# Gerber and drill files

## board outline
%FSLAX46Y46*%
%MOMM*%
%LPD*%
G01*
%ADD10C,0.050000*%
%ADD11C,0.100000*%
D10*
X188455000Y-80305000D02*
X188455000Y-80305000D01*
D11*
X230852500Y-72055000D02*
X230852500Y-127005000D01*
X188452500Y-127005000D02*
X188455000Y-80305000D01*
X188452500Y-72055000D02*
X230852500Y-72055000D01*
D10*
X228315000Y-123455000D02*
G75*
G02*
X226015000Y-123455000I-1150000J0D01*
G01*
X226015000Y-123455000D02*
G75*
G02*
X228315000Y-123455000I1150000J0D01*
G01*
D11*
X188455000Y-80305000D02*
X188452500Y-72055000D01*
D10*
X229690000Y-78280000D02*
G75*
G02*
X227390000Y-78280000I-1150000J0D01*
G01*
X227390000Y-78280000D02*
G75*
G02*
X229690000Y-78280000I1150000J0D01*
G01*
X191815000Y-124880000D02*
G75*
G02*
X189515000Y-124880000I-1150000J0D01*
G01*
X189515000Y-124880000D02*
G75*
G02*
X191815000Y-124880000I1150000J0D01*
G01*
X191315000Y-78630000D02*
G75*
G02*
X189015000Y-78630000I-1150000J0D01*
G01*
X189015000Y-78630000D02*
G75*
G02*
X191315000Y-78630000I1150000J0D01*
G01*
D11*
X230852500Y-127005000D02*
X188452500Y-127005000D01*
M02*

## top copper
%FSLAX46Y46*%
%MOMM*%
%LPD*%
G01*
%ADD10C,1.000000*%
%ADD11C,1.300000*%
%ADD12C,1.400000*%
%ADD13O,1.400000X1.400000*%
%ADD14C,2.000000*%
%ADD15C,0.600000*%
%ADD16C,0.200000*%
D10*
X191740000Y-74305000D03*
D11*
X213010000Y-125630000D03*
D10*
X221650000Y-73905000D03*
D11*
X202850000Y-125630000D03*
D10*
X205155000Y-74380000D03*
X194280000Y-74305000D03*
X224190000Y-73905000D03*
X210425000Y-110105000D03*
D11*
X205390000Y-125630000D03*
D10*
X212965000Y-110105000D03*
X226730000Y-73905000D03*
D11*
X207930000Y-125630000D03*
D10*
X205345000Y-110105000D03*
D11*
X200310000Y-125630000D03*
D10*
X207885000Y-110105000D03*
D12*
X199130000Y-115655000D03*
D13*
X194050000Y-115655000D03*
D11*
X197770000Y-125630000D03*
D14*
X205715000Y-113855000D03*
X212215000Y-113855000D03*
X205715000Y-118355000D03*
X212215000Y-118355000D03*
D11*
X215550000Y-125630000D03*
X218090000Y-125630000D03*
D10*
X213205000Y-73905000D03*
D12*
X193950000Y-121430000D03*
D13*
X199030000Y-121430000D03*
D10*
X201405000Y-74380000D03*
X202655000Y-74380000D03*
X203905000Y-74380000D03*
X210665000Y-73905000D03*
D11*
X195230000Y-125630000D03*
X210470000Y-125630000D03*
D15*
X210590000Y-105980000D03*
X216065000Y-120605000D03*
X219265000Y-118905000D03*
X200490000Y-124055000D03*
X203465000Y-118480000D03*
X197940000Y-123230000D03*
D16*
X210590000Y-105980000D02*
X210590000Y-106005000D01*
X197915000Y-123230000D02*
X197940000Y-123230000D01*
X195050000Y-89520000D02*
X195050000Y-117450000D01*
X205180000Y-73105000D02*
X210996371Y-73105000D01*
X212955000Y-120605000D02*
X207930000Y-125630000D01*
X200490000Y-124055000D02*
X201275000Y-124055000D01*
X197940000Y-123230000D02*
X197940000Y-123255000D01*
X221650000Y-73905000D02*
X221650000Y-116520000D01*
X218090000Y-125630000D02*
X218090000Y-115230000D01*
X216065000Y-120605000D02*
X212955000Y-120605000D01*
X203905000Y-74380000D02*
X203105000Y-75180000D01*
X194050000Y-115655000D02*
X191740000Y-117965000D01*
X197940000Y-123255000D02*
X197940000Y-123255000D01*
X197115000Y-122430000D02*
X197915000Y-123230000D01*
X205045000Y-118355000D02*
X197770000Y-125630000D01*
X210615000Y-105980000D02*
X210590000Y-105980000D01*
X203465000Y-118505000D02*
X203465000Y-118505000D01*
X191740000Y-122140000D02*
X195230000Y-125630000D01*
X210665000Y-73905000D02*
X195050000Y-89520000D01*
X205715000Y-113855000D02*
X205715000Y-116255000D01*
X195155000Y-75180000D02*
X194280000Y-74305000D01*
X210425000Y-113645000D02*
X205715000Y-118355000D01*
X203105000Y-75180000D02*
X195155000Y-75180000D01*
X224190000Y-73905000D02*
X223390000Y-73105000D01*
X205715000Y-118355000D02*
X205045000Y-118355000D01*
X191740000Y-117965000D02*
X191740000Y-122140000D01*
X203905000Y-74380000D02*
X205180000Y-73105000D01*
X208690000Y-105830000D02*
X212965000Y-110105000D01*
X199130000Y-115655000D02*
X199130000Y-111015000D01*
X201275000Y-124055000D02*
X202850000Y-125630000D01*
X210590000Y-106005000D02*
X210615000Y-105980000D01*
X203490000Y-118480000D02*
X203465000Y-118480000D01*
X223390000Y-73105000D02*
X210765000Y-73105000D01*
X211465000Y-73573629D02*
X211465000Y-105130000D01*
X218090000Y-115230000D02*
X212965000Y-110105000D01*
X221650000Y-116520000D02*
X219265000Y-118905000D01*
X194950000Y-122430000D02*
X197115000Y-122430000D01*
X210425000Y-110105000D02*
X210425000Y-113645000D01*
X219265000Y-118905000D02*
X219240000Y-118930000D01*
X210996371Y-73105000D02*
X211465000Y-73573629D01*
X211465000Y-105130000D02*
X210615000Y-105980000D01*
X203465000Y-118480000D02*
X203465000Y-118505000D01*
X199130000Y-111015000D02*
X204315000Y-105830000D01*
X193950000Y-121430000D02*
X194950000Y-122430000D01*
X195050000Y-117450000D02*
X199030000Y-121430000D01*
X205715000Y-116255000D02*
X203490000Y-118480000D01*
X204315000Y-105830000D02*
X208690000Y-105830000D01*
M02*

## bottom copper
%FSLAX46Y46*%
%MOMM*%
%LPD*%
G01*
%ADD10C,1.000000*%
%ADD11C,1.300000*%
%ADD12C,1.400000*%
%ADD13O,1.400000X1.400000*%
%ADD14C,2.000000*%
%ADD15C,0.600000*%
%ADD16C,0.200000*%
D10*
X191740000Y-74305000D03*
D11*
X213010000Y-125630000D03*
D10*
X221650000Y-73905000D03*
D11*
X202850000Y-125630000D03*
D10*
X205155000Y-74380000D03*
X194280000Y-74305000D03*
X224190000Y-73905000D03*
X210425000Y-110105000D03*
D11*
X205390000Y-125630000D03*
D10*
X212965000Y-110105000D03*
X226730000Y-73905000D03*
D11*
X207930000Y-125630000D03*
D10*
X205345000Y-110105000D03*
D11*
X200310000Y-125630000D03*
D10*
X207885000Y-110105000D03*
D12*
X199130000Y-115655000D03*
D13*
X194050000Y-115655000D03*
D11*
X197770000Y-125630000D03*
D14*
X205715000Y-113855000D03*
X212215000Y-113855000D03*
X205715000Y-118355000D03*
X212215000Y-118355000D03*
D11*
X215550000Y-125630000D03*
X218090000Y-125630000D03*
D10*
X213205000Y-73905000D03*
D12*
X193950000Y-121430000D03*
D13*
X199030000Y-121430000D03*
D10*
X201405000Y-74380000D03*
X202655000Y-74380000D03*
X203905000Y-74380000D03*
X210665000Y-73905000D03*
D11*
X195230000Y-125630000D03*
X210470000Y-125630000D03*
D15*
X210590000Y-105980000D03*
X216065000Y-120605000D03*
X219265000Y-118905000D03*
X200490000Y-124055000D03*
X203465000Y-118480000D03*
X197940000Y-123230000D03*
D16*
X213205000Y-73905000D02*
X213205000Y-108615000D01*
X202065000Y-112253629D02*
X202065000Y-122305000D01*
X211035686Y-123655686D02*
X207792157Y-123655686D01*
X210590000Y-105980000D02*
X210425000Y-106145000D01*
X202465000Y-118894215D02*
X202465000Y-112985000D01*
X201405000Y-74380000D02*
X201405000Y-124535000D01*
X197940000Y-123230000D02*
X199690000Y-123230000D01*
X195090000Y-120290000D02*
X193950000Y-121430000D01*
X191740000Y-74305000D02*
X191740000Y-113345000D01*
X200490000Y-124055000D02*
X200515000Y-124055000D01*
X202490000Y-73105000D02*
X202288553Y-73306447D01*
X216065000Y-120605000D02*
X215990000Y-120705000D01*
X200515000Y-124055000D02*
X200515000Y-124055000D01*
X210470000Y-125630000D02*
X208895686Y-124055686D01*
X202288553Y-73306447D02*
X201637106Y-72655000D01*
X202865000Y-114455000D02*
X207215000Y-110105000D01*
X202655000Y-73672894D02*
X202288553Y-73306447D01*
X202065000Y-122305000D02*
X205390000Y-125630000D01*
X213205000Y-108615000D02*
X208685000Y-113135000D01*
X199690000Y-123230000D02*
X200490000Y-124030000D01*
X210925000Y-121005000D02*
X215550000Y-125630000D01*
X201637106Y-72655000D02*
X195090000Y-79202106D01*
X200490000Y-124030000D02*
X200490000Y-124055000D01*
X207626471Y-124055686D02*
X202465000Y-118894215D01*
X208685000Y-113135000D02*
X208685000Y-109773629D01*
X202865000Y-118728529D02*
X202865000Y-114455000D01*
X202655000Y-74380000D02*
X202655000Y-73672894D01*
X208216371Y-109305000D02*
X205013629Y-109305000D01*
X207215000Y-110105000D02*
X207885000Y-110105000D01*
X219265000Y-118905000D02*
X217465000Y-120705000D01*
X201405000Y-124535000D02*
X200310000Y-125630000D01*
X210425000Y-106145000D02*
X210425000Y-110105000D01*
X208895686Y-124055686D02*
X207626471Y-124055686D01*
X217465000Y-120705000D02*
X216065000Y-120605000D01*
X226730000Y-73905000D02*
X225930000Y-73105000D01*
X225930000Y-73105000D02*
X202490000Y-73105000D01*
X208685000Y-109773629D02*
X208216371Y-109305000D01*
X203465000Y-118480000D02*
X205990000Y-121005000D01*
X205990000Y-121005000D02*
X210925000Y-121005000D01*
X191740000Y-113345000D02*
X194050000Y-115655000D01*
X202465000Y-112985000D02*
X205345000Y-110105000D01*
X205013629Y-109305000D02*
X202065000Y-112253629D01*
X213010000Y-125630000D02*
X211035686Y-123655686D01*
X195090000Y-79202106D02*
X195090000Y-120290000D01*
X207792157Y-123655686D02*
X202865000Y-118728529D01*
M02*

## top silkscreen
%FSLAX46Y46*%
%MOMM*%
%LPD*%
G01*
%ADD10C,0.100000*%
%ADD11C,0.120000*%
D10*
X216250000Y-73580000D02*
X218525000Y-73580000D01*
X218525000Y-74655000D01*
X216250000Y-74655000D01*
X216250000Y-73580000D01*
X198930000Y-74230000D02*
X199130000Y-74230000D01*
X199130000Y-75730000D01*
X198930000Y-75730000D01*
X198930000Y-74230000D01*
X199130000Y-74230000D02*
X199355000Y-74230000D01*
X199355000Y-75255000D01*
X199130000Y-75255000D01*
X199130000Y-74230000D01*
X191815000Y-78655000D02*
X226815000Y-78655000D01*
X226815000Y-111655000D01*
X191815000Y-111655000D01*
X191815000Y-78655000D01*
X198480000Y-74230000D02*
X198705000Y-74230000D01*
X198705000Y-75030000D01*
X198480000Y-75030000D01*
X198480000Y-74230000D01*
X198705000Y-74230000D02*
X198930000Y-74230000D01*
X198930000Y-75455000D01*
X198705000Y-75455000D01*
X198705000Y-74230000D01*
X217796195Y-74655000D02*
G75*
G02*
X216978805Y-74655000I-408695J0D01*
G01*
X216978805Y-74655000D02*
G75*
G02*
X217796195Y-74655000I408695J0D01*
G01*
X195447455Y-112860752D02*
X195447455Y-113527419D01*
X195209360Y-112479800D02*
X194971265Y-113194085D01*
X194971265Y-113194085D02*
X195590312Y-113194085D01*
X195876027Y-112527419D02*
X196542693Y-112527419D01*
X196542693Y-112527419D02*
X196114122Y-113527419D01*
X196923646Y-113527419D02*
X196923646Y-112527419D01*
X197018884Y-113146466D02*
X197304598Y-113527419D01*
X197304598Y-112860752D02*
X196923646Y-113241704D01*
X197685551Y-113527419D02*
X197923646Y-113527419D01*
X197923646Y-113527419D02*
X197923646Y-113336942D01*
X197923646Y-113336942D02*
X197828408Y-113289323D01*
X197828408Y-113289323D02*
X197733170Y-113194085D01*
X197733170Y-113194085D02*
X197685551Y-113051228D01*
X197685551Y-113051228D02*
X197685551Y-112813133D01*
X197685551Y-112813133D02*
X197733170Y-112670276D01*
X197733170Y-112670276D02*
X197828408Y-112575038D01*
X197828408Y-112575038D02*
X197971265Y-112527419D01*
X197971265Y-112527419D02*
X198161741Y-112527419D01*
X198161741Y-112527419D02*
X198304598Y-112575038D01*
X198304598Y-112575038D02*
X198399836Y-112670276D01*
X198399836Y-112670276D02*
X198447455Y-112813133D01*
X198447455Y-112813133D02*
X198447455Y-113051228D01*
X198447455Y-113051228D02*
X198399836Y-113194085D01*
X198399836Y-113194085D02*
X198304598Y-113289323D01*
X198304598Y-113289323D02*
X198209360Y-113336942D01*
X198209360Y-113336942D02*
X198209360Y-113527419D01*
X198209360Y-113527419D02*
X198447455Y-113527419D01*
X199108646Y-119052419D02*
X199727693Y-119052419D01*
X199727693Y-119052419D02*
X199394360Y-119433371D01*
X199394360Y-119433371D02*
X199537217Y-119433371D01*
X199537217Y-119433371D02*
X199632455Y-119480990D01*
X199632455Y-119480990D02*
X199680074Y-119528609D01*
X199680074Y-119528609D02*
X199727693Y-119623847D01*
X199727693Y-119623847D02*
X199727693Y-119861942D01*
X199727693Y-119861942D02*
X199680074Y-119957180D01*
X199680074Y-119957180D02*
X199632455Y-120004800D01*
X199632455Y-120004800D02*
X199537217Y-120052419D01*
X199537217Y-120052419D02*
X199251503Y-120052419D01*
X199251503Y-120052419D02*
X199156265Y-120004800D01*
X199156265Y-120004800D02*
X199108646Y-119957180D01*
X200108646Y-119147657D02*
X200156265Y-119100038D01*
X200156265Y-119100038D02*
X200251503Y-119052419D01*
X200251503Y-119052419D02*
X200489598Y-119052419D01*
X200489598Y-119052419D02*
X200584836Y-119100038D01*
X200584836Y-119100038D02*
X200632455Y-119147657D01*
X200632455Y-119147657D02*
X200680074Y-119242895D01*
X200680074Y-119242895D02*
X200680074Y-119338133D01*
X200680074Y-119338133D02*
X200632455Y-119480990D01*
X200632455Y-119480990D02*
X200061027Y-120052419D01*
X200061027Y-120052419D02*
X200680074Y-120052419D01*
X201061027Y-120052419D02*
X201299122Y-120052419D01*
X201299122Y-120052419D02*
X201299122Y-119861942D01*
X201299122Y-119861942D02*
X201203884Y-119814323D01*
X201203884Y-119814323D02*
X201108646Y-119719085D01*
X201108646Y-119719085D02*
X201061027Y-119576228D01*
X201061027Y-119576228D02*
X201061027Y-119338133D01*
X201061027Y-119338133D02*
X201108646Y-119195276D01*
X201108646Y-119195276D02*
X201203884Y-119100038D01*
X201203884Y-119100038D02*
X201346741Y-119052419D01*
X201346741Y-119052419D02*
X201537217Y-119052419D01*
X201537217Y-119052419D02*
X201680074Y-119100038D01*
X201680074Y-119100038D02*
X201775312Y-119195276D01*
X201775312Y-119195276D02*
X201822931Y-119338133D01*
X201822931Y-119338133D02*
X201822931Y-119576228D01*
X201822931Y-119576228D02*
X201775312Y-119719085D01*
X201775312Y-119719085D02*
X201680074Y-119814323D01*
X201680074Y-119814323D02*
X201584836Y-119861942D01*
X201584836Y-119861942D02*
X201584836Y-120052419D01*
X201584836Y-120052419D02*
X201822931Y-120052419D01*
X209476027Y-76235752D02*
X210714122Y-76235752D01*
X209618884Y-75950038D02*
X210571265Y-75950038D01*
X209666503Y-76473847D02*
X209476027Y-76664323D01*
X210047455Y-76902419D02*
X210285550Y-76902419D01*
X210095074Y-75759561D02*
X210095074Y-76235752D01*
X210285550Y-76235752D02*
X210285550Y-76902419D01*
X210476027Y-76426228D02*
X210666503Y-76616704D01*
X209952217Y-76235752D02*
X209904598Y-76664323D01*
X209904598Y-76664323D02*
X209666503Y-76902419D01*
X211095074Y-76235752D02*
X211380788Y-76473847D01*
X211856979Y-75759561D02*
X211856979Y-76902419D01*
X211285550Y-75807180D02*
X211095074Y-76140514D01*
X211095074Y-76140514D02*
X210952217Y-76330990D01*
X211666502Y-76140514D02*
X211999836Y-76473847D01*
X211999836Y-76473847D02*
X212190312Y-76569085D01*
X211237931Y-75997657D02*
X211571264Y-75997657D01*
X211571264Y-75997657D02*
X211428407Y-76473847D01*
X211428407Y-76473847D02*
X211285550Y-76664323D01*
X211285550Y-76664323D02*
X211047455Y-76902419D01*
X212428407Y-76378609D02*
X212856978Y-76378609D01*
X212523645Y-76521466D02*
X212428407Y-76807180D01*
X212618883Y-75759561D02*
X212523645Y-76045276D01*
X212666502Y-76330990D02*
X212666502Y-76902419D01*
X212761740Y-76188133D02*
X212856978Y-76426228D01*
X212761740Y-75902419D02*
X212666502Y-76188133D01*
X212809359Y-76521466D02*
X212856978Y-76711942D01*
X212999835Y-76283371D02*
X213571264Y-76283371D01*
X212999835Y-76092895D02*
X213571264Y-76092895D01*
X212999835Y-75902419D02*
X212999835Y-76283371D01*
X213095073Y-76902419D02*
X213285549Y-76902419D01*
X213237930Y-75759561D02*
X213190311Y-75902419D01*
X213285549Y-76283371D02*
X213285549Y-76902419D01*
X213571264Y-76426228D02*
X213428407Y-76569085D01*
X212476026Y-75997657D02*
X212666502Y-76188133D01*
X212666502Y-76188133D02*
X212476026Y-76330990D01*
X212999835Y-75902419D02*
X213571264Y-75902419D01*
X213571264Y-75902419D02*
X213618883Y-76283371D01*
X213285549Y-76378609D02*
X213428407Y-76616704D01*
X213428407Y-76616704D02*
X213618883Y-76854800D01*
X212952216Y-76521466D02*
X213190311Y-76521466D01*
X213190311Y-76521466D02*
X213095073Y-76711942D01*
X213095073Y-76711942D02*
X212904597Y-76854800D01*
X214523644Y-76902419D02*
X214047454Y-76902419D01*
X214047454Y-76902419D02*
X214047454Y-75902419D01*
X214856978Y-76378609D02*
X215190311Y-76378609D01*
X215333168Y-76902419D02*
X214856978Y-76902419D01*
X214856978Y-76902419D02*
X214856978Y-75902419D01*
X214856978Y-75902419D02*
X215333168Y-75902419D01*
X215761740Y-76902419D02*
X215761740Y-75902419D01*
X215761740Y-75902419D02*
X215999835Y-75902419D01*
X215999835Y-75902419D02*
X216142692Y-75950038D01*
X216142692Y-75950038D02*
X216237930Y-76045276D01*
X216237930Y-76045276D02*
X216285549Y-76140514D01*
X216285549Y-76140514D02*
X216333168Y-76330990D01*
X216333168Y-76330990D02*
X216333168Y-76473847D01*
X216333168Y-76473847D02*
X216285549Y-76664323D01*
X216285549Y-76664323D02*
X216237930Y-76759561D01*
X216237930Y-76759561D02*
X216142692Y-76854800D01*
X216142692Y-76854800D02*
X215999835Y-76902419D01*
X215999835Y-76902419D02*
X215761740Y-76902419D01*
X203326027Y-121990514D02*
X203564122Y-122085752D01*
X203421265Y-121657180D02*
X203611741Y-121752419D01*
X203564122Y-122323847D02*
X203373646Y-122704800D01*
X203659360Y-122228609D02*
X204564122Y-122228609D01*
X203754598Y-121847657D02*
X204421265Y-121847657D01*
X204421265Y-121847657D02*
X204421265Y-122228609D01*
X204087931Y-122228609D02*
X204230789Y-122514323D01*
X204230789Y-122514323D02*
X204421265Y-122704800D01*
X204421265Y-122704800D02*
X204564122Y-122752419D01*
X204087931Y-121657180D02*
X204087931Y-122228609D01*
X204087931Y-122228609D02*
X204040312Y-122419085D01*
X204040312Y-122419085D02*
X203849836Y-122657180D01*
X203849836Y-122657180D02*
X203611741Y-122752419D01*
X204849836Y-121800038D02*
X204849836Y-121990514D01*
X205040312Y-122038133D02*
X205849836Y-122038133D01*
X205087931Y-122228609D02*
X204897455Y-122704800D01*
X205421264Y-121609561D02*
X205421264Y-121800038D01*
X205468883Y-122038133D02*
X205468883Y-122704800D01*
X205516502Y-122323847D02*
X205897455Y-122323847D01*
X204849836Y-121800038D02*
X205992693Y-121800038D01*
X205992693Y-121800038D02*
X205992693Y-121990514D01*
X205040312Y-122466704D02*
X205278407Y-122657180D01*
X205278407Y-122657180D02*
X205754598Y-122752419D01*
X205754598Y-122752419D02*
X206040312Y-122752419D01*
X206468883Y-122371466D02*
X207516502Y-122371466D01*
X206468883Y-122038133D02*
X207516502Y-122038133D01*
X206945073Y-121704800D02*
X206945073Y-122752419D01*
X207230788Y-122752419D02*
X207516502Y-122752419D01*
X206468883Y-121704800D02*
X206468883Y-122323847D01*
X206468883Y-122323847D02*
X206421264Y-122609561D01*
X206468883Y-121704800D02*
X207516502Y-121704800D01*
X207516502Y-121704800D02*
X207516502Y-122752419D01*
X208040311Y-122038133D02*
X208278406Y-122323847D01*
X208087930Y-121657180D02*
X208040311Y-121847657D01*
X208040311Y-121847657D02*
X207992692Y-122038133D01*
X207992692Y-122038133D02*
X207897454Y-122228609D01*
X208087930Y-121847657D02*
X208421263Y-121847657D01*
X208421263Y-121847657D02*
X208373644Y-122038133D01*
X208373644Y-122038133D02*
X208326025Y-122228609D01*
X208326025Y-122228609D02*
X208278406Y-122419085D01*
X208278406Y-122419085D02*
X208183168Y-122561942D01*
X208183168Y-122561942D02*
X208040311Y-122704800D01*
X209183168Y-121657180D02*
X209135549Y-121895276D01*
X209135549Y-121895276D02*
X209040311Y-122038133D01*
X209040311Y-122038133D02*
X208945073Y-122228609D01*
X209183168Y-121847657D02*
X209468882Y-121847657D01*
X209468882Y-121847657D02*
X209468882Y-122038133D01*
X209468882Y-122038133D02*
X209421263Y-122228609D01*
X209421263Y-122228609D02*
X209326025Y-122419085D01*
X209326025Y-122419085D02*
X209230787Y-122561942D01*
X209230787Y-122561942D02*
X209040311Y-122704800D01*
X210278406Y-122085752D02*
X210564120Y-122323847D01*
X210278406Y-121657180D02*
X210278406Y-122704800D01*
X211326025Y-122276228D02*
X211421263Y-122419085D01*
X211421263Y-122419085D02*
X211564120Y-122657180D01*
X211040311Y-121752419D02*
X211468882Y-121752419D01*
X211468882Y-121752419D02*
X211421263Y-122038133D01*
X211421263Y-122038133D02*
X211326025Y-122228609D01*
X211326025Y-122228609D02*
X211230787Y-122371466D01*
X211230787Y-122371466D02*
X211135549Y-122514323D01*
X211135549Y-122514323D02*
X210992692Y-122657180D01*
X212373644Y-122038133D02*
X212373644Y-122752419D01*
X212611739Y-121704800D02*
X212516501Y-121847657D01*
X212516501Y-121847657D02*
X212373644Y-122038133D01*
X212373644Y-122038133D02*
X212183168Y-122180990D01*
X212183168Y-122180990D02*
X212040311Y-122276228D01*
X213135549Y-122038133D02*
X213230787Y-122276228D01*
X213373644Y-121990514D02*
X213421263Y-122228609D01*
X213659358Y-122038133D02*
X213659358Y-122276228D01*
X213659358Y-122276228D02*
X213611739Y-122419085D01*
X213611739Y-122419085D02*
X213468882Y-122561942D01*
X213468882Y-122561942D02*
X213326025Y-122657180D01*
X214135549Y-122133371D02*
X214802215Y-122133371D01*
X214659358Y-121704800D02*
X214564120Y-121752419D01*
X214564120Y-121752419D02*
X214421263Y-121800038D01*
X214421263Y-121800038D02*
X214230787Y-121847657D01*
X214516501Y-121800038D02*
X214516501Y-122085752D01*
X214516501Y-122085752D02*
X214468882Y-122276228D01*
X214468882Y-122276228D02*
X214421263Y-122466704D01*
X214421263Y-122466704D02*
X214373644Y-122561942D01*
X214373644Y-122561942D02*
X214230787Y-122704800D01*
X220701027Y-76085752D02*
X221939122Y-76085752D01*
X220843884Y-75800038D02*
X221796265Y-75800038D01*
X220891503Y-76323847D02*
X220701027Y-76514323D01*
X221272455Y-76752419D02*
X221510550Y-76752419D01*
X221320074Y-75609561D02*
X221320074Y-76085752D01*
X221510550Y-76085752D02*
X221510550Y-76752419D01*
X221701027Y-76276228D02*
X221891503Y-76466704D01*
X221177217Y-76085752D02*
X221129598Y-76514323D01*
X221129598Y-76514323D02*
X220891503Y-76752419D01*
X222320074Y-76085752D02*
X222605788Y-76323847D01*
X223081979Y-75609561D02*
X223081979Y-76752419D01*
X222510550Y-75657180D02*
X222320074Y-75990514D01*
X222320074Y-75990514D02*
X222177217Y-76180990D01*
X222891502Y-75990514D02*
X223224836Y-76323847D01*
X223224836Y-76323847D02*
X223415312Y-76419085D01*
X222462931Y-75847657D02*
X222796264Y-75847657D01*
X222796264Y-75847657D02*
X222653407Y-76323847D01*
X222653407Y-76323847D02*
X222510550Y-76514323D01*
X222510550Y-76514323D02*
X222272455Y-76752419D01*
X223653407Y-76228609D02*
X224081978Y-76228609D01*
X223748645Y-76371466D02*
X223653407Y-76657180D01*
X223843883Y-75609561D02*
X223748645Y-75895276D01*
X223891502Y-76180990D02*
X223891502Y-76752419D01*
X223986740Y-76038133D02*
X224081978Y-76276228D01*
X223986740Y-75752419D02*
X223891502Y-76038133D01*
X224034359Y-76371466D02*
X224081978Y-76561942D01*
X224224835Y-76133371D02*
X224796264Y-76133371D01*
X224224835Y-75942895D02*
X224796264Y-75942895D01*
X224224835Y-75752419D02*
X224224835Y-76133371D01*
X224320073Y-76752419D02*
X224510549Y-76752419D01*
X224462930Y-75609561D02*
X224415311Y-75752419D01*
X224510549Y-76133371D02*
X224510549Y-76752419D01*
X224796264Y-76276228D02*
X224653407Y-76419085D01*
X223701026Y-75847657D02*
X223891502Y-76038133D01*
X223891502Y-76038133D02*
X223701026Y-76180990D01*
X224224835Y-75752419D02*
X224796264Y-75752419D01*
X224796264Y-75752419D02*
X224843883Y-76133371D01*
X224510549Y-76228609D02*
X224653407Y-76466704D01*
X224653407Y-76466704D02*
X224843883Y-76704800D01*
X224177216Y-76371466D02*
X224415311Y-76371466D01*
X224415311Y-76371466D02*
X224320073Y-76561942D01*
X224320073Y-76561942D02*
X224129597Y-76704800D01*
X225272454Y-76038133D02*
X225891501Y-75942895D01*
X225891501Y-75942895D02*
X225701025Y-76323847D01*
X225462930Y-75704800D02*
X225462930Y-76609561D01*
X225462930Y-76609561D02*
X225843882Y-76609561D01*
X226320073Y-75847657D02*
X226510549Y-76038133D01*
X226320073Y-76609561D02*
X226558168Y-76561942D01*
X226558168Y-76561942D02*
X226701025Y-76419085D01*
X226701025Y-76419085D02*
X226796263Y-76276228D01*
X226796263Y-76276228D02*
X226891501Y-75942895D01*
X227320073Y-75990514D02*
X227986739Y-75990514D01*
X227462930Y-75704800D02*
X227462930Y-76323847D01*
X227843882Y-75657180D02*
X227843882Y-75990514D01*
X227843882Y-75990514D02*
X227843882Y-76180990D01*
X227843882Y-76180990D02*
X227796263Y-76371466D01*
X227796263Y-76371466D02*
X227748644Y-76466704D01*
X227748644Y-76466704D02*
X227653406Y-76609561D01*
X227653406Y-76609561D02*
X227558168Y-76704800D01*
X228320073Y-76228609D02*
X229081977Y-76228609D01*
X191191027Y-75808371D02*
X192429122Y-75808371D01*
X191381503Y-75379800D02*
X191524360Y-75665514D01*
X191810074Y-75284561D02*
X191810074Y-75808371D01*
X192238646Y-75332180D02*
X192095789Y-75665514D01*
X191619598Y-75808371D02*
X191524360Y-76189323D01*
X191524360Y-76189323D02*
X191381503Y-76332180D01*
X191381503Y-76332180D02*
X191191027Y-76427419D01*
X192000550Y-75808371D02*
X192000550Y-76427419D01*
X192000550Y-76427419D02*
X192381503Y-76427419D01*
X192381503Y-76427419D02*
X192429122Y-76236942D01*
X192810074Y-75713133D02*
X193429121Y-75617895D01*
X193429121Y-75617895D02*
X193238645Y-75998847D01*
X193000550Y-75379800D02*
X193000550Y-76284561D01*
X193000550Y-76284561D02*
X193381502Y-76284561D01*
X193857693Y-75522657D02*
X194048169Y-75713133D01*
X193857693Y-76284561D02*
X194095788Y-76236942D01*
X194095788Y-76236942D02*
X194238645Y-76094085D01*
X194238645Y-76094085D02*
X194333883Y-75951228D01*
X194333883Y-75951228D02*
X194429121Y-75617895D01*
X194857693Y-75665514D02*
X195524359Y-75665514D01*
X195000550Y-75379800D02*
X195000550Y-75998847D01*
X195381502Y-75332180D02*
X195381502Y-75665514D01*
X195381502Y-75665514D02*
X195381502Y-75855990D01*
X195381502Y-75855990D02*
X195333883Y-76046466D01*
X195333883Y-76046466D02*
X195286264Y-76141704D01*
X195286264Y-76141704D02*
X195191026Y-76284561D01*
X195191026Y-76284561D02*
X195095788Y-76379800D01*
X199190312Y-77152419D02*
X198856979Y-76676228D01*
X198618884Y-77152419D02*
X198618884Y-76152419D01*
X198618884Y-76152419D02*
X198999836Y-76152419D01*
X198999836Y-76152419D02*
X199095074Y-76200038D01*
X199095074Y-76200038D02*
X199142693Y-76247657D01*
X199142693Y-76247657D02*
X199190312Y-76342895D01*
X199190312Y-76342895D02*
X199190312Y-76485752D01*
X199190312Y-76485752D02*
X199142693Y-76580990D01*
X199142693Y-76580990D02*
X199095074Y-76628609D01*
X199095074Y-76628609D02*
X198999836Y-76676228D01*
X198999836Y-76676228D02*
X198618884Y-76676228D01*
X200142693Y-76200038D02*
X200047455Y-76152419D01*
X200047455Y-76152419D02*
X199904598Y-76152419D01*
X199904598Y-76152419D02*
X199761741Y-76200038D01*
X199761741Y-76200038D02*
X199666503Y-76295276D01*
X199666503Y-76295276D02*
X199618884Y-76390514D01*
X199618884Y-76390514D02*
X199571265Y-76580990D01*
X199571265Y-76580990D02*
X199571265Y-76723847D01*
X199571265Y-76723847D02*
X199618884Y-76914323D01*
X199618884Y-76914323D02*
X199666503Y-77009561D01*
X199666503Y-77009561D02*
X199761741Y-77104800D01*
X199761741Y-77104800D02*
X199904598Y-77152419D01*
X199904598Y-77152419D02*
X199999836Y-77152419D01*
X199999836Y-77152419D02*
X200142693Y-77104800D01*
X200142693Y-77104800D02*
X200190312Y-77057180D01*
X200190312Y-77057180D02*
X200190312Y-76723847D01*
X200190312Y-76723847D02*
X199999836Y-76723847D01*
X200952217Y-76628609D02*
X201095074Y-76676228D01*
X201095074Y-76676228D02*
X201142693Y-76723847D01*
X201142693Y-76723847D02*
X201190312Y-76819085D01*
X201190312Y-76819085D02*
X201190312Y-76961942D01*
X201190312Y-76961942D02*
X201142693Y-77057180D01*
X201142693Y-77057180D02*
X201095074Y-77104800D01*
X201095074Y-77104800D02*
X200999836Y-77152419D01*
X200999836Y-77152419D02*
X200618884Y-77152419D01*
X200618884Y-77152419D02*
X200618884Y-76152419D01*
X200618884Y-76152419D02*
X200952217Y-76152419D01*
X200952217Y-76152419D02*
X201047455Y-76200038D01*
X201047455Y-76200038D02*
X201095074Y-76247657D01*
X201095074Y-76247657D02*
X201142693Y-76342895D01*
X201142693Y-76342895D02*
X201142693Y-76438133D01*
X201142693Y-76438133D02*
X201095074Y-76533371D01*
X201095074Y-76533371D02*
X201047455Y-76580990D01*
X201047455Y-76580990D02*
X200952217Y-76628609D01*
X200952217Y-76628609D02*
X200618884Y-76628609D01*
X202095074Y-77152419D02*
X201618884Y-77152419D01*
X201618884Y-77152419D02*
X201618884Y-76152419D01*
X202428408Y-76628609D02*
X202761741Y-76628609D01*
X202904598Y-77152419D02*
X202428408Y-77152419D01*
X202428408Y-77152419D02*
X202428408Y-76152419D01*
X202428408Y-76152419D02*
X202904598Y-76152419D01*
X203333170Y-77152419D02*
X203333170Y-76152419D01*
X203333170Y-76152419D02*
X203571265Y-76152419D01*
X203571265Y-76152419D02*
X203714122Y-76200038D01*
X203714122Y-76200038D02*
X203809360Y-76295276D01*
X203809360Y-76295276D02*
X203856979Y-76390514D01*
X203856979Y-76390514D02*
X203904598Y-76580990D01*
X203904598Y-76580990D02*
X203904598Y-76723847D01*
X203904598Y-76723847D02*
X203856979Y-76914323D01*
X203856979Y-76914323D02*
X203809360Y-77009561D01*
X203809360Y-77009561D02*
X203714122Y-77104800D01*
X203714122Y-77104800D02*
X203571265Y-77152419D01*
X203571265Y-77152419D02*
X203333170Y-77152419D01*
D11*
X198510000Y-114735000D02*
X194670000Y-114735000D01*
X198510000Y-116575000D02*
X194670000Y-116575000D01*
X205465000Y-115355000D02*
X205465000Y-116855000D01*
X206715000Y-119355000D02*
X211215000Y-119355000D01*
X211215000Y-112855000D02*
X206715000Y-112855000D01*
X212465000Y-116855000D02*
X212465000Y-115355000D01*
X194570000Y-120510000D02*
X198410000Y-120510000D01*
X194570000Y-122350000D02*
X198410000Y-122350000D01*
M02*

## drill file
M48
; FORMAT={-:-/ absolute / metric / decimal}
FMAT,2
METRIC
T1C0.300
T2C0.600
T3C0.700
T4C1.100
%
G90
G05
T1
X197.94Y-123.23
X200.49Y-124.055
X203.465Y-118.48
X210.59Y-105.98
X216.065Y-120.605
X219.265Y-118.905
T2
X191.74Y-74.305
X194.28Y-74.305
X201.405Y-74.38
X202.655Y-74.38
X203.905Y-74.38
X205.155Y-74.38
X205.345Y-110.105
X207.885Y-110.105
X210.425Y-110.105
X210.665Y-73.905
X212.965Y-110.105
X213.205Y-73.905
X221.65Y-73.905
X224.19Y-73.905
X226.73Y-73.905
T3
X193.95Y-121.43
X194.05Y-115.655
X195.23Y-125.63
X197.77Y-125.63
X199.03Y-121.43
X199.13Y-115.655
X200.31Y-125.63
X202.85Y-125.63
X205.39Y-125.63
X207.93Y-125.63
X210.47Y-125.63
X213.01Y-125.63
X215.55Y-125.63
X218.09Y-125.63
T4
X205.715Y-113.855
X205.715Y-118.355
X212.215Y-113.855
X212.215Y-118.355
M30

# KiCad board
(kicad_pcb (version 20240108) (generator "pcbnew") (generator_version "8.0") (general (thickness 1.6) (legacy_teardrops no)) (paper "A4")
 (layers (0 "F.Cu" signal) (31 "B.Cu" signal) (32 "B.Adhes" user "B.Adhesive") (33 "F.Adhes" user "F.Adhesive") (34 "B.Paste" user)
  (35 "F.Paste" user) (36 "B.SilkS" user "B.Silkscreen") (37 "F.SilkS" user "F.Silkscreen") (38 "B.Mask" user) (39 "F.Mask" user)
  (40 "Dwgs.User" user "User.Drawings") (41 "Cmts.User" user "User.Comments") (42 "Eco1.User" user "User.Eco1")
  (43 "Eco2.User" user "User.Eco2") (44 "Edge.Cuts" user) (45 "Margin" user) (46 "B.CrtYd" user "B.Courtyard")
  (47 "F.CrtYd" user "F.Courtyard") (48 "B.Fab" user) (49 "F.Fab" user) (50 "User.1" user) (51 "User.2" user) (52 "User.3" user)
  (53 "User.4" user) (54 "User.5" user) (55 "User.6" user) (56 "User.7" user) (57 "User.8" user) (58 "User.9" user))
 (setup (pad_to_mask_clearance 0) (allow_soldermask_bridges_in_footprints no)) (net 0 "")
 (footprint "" (layer "F.Cu") (at 191.74 74.305)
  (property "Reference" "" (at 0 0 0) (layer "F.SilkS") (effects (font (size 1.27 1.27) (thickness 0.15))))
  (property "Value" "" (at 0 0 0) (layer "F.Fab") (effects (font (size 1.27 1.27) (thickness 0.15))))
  (pad "" thru_hole circle (at 0 0 180) (size 1 1) (drill 0.6) (layers "*.Cu" "*.Mask") (remove_unused_layers no)))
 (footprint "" (layer "F.Cu") (at 213.01 125.63)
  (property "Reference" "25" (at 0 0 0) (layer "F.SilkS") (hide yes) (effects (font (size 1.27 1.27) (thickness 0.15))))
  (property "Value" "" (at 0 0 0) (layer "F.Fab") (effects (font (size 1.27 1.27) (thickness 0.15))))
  (pad "" thru_hole circle (at 0 0 180) (size 1.3 1.3) (drill 0.7) (layers "*.Cu" "*.Mask") (remove_unused_layers no)))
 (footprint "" (layer "F.Cu") (at 221.65 73.905)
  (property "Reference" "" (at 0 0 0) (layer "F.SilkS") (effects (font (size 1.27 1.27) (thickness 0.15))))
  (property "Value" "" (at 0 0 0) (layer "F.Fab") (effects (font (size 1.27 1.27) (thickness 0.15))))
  (pad "" thru_hole circle (at 0 0 180) (size 1 1) (drill 0.6) (layers "*.Cu" "*.Mask") (remove_unused_layers no)))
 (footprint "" (layer "F.Cu") (at 202.85 125.63)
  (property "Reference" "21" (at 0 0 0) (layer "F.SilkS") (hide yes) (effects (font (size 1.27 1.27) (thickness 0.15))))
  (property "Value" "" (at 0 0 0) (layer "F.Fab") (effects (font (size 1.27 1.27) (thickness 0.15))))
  (pad "" thru_hole circle (at 0 0 180) (size 1.3 1.3) (drill 0.7) (layers "*.Cu" "*.Mask") (remove_unused_layers no)))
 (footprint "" (layer "F.Cu") (at 205.155 74.38)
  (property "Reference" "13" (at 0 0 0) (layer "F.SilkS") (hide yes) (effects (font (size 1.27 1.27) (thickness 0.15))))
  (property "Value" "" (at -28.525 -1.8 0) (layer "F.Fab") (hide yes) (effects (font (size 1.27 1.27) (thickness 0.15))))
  (pad "" thru_hole circle (at 0 0 180) (size 1 1) (drill 0.6) (layers "*.Cu" "*.Mask") (remove_unused_layers no)))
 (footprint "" (layer "F.Cu") (at 194.28 74.305)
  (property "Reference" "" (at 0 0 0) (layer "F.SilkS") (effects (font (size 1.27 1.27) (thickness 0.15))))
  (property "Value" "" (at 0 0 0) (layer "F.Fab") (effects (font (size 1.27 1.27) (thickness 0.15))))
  (pad "" thru_hole circle (at 0 0 180) (size 1 1) (drill 0.6) (layers "*.Cu" "*.Mask") (remove_unused_layers no)))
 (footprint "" (layer "F.Cu") (at 224.19 73.905)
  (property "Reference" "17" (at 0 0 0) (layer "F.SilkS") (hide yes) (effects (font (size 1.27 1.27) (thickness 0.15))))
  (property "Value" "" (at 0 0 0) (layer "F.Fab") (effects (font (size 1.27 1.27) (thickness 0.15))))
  (pad "" thru_hole circle (at 0 0 180) (size 1 1) (drill 0.6) (layers "*.Cu" "*.Mask") (remove_unused_layers no)))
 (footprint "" (layer "F.Cu") (at 210.425 110.105)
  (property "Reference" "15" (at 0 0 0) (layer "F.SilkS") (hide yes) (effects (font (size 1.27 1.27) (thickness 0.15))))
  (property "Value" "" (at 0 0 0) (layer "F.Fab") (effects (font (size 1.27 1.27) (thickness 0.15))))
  (pad "" thru_hole circle (at 0 0 180) (size 1 1) (drill 0.6) (layers "*.Cu" "*.Mask") (remove_unused_layers no)))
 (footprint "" (layer "F.Cu") (at 205.39 125.63)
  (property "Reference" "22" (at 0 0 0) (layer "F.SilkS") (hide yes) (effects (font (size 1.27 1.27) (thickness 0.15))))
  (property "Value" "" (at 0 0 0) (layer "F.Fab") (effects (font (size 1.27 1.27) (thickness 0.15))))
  (pad "e" thru_hole circle (at 0 0 180) (size 1.3 1.3) (drill 0.7) (layers "*.Cu" "*.Mask") (remove_unused_layers no)))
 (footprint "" (layer "F.Cu") (at 212.965 110.105)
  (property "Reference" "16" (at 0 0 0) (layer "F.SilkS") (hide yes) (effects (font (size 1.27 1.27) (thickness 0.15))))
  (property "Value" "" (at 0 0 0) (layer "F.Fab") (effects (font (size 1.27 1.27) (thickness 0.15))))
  (pad "" thru_hole circle (at 0 0 180) (size 1 1) (drill 0.6) (layers "*.Cu" "*.Mask") (remove_unused_layers no)))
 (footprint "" (layer "F.Cu") (at 226.73 73.905)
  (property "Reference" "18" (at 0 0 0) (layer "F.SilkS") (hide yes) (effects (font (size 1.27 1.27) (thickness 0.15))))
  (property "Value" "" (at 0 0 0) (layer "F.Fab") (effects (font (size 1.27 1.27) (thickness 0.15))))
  (pad "" thru_hole circle (at 0 0 180) (size 1 1) (drill 0.6) (layers "*.Cu" "*.Mask") (remove_unused_layers no)))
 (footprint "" (layer "F.Cu") (at 207.93 125.63)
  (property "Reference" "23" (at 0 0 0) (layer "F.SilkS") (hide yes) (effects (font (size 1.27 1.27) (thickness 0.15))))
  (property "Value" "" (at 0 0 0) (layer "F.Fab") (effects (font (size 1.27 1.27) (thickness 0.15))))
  (pad "" thru_hole circle (at 0 0 180) (size 1.3 1.3) (drill 0.7) (layers "*.Cu" "*.Mask") (remove_unused_layers no)))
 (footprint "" (layer "F.Cu") (at 205.345 110.105)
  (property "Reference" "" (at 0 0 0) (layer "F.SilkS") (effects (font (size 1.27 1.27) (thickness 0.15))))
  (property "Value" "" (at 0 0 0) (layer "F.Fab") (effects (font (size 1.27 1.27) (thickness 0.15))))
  (pad "" thru_hole circle (at 0 0 180) (size 1 1) (drill 0.6) (layers "*.Cu" "*.Mask") (remove_unused_layers no)))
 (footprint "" (layer "F.Cu") (at 200.31 125.63)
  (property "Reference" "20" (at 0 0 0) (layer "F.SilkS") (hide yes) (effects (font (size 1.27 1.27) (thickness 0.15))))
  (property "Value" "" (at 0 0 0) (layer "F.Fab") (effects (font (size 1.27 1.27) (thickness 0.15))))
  (pad "" thru_hole circle (at 0 0 180) (size 1.3 1.3) (drill 0.7) (layers "*.Cu" "*.Mask") (remove_unused_layers no)))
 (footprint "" (layer "F.Cu") (at 207.885 110.105)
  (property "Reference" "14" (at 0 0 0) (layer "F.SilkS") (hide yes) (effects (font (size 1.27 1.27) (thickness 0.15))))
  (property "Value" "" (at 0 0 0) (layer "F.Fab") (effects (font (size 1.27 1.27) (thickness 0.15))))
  (pad "" thru_hole circle (at 0 0 180) (size 1 1) (drill 0.6) (layers "*.Cu" "*.Mask") (remove_unused_layers no)))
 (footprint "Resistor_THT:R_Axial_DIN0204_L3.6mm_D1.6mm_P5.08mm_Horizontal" (layer "F.Cu") (at 199.13 115.655 180)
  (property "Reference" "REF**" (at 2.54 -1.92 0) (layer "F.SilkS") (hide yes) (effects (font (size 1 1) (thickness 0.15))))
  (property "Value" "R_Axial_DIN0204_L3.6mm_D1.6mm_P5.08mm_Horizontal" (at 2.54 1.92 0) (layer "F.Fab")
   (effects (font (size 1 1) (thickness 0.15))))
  (fp_line (start 0.62 0.92) (end 4.46 0.92) (stroke (width 0.12) (type solid)) (layer "F.SilkS"))
  (fp_line (start 0.62 -0.92) (end 4.46 -0.92) (stroke (width 0.12) (type solid)) (layer "F.SilkS"))
  (pad "1" thru_hole circle (at 0 0 180) (size 1.4 1.4) (drill 0.7) (layers "*.Cu" "*.Mask") (remove_unused_layers no))
  (pad "2" thru_hole oval (at 5.08 0 180) (size 1.4 1.4) (drill 0.7) (layers "*.Cu" "*.Mask") (remove_unused_layers no)))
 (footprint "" (layer "F.Cu") (at 197.77 125.63)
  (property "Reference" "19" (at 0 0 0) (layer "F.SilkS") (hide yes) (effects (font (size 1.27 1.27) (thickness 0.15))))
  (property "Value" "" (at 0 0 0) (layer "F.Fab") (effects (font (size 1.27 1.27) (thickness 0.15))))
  (pad "" thru_hole circle (at 0 0 180) (size 1.3 1.3) (drill 0.7) (layers "*.Cu" "*.Mask") (remove_unused_layers no)))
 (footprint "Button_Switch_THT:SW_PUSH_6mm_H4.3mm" (layer "F.Cu") (at 205.715 113.855)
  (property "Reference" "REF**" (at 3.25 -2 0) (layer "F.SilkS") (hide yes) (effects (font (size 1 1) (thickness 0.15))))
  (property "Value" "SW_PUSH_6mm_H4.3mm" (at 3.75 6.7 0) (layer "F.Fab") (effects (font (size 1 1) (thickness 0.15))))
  (fp_line (start -0.25 1.5) (end -0.25 3) (stroke (width 0.12) (type solid)) (layer "F.SilkS"))
  (fp_line (start 1 5.5) (end 5.5 5.5) (stroke (width 0.12) (type solid)) (layer "F.SilkS"))
  (fp_line (start 5.5 -1) (end 1 -1) (stroke (width 0.12) (type solid)) (layer "F.SilkS"))
  (fp_line (start 6.75 3) (end 6.75 1.5) (stroke (width 0.12) (type solid)) (layer "F.SilkS"))
  (pad "1" thru_hole circle (at 0 0 90) (size 2 2) (drill 1.1) (layers "*.Cu" "*.Mask") (remove_unused_layers no))
  (pad "1" thru_hole circle (at 6.5 0 90) (size 2 2) (drill 1.1) (layers "*.Cu" "*.Mask") (remove_unused_layers no))
  (pad "2" thru_hole circle (at 0 4.5 90) (size 2 2) (drill 1.1) (layers "*.Cu" "*.Mask") (remove_unused_layers no))
  (pad "2" thru_hole circle (at 6.5 4.5 90) (size 2 2) (drill 1.1) (layers "*.Cu" "*.Mask") (remove_unused_layers no)))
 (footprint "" (layer "F.Cu") (at 215.55 125.63)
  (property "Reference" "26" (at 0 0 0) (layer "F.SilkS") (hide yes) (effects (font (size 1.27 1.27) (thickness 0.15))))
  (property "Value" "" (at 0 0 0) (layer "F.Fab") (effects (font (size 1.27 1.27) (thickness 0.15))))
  (pad "" thru_hole circle (at 0 0 180) (size 1.3 1.3) (drill 0.7) (layers "*.Cu" "*.Mask") (remove_unused_layers no)))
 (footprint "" (layer "F.Cu") (at 218.09 125.63)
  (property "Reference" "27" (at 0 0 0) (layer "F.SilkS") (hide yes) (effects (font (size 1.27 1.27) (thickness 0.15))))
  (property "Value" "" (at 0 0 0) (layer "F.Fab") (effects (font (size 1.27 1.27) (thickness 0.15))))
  (pad "" thru_hole circle (at 0 0 180) (size 1.3 1.3) (drill 0.7) (layers "*.Cu" "*.Mask") (remove_unused_layers no)))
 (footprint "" (layer "F.Cu") (at 213.205 73.905)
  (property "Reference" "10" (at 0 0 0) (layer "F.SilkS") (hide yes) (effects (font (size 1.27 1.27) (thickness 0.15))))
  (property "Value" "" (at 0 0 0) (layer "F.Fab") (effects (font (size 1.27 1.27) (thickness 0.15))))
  (pad "" thru_hole circle (at 0 0 180) (size 1 1) (drill 0.6) (layers "*.Cu" "*.Mask") (remove_unused_layers no)))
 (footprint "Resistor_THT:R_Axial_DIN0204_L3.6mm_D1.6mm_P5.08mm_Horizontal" (layer "F.Cu") (at 193.95 121.43)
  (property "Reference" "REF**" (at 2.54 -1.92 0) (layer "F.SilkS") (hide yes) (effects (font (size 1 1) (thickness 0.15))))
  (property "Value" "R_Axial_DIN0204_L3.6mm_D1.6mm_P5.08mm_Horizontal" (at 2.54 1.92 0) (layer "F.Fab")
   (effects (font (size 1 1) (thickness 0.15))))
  (fp_line (start 0.62 -0.92) (end 4.46 -0.92) (stroke (width 0.12) (type solid)) (layer "F.SilkS"))
  (fp_line (start 0.62 0.92) (end 4.46 0.92) (stroke (width 0.12) (type solid)) (layer "F.SilkS"))
  (pad "1" thru_hole circle (at 0 0) (size 1.4 1.4) (drill 0.7) (layers "*.Cu" "*.Mask") (remove_unused_layers no))
  (pad "2" thru_hole oval (at 5.08 0) (size 1.4 1.4) (drill 0.7) (layers "*.Cu" "*.Mask") (remove_unused_layers no)))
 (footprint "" (layer "F.Cu") (at 201.405 74.38)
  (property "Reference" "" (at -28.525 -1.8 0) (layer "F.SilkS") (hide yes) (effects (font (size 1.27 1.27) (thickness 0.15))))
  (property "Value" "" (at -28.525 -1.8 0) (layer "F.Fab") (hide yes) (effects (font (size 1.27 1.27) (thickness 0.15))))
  (pad "" thru_hole circle (at 0 0 180) (size 1 1) (drill 0.6) (layers "*.Cu" "*.Mask") (remove_unused_layers no)))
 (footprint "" (layer "F.Cu") (at 202.655 74.38)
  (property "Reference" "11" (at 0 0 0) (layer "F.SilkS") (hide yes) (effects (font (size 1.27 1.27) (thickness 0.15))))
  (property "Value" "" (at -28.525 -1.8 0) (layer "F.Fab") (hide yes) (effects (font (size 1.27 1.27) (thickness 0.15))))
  (pad "" thru_hole circle (at 0 0 180) (size 1 1) (drill 0.6) (layers "*.Cu" "*.Mask") (remove_unused_layers no)))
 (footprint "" (layer "F.Cu") (at 203.905 74.38)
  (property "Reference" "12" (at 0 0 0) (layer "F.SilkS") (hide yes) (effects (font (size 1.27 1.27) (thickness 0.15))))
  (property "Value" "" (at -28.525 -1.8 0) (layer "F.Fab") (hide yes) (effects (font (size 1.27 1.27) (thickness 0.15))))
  (pad "" thru_hole circle (at 0 0 180) (size 1 1) (drill 0.6) (layers "*.Cu" "*.Mask") (remove_unused_layers no)))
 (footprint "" (layer "F.Cu") (at 210.665 73.905)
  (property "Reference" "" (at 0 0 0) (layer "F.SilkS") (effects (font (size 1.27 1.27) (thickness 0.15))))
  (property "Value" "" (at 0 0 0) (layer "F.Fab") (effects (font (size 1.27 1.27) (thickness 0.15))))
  (pad "" thru_hole circle (at 0 0 180) (size 1 1) (drill 0.6) (layers "*.Cu" "*.Mask") (remove_unused_layers no)))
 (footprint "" (layer "F.Cu") (at 195.23 125.63)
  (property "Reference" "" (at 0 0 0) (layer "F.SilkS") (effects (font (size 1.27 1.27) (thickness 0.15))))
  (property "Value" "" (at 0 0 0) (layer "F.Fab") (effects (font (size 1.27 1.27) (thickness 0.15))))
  (pad "" thru_hole circle (at 0 0 180) (size 1.3 1.3) (drill 0.7) (layers "*.Cu" "*.Mask") (remove_unused_layers no)))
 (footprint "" (layer "F.Cu") (at 210.47 125.63)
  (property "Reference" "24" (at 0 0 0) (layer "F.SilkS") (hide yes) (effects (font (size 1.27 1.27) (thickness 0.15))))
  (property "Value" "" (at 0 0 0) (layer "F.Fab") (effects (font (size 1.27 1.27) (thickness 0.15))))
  (pad "" thru_hole circle (at 0 0 180) (size 1.3 1.3) (drill 0.7) (layers "*.Cu" "*.Mask") (remove_unused_layers no)))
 (gr_rect (start 216.25 73.58) (end 218.525 74.655) (stroke (width 0.1) (type default)) (fill none) (layer "F.SilkS"))
 (gr_rect (start 198.93 74.23) (end 199.13 75.73) (stroke (width 0.1) (type default)) (fill none) (layer "F.SilkS"))
 (gr_rect (start 199.13 74.23) (end 199.355 75.255) (stroke (width 0.1) (type default)) (fill none) (layer "F.SilkS"))
 (gr_rect (start 191.815 78.655) (end 226.815 111.655) (stroke (width 0.1) (type default)) (fill none) (layer "F.SilkS"))
 (gr_rect (start 198.48 74.23) (end 198.705 75.03) (stroke (width 0.1) (type default)) (fill none) (layer "F.SilkS"))
 (gr_rect (start 198.705 74.23) (end 198.93 75.455) (stroke (width 0.1) (type default)) (fill none) (layer "F.SilkS"))
 (gr_circle (center 217.3875 74.655) (end 217.55 74.28) (stroke (width 0.1) (type default)) (fill none) (layer "F.SilkS"))
 (gr_line (start 188.455 80.305) (end 188.455 80.305) (stroke (width 0.05) (type default)) (layer "Edge.Cuts"))
 (gr_line (start 230.8525 72.055) (end 230.8525 127.005) (stroke (width 0.1) (type default)) (layer "Edge.Cuts"))
 (gr_line (start 188.4525 127.005) (end 188.455 80.305) (stroke (width 0.1) (type default)) (layer "Edge.Cuts"))
 (gr_line (start 188.4525 72.055) (end 230.8525 72.055) (stroke (width 0.1) (type default)) (layer "Edge.Cuts"))
 (gr_circle (center 227.165 123.455) (end 226.015 123.455) (stroke (width 0.05) (type default)) (fill none) (layer "Edge.Cuts"))
 (gr_line (start 188.455 80.305) (end 188.4525 72.055) (stroke (width 0.1) (type default)) (layer "Edge.Cuts"))
 (gr_circle (center 228.54 78.28) (end 227.39 78.28) (stroke (width 0.05) (type default)) (fill none) (layer "Edge.Cuts"))
 (gr_circle (center 190.665 124.88) (end 189.515 124.88) (stroke (width 0.05) (type default)) (fill none) (layer "Edge.Cuts"))
 (gr_circle (center 190.165 78.63) (end 189.015 78.63) (stroke (width 0.05) (type default)) (fill none) (layer "Edge.Cuts"))
 (gr_line (start 230.8525 127.005) (end 188.4525 127.005) (stroke (width 0.1) (type default)) (layer "Edge.Cuts"))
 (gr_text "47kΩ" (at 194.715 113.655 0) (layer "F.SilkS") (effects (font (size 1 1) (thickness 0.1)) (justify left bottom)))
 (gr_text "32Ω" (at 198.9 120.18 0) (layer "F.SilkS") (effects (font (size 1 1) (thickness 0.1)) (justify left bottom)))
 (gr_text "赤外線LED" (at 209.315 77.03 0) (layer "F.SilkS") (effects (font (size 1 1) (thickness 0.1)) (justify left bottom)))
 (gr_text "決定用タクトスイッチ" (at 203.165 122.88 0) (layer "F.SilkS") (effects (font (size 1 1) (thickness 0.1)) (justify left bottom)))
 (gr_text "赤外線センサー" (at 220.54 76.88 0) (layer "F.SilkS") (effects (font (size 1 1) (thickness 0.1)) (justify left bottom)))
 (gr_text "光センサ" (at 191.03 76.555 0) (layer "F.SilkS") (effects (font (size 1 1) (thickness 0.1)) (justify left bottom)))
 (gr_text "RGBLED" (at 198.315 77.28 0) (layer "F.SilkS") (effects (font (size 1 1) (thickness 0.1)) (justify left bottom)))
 (segment (start 210.59 105.98) (end 210.59 106.005) (width 0.2) (layer "F.Cu") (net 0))
 (segment (start 197.915 123.23) (end 197.94 123.23) (width 0.2) (layer "F.Cu") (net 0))
 (segment (start 195.05 89.52) (end 195.05 117.45) (width 0.2) (layer "F.Cu") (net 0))
 (segment (start 205.18 73.105) (end 210.996371 73.105) (width 0.2) (layer "F.Cu") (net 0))
 (segment (start 212.955 120.605) (end 207.93 125.63) (width 0.2) (layer "F.Cu") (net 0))
 (segment (start 200.49 124.055) (end 201.275 124.055) (width 0.2) (layer "F.Cu") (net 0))
 (segment (start 197.94 123.23) (end 197.94 123.255) (width 0.2) (layer "F.Cu") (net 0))
 (segment (start 221.65 73.905) (end 221.65 116.52) (width 0.2) (layer "F.Cu") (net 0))
 (segment (start 218.09 125.63) (end 218.09 115.23) (width 0.2) (layer "F.Cu") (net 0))
 (segment (start 216.065 120.605) (end 212.955 120.605) (width 0.2) (layer "F.Cu") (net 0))
 (segment (start 203.905 74.38) (end 203.105 75.18) (width 0.2) (layer "F.Cu") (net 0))
 (segment (start 194.05 115.655) (end 191.74 117.965) (width 0.2) (layer "F.Cu") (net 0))
 (segment (start 197.94 123.255) (end 197.94 123.255) (width 0.2) (layer "F.Cu") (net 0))
 (segment (start 197.115 122.43) (end 197.915 123.23) (width 0.2) (layer "F.Cu") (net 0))
 (segment (start 205.045 118.355) (end 197.77 125.63) (width 0.2) (layer "F.Cu") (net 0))
 (segment (start 210.615 105.98) (end 210.59 105.98) (width 0.2) (layer "F.Cu") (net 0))
 (segment (start 203.465 118.505) (end 203.465 118.505) (width 0.2) (layer "F.Cu") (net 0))
 (segment (start 191.74 122.14) (end 195.23 125.63) (width 0.2) (layer "F.Cu") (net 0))
 (segment (start 210.665 73.905) (end 195.05 89.52) (width 0.2) (layer "F.Cu") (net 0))
 (segment (start 205.715 113.855) (end 205.715 116.255) (width 0.2) (layer "F.Cu") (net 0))
 (segment (start 195.155 75.18) (end 194.28 74.305) (width 0.2) (layer "F.Cu") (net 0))
 (segment (start 210.425 113.645) (end 205.715 118.355) (width 0.2) (layer "F.Cu") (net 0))
 (segment (start 203.105 75.18) (end 195.155 75.18) (width 0.2) (layer "F.Cu") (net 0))
 (segment (start 224.19 73.905) (end 223.39 73.105) (width 0.2) (layer "F.Cu") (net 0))
 (segment (start 205.715 118.355) (end 205.045 118.355) (width 0.2) (layer "F.Cu") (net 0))
 (segment (start 191.74 117.965) (end 191.74 122.14) (width 0.2) (layer "F.Cu") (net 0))
 (segment (start 203.905 74.38) (end 205.18 73.105) (width 0.2) (layer "F.Cu") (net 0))
 (segment (start 208.69 105.83) (end 212.965 110.105) (width 0.2) (layer "F.Cu") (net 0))
 (segment (start 199.13 115.655) (end 199.13 111.015) (width 0.2) (layer "F.Cu") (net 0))
 (segment (start 201.275 124.055) (end 202.85 125.63) (width 0.2) (layer "F.Cu") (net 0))
 (segment (start 210.59 106.005) (end 210.615 105.98) (width 0.2) (layer "F.Cu") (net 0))
 (segment (start 203.49 118.48) (end 203.465 118.48) (width 0.2) (layer "F.Cu") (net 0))
 (segment (start 223.39 73.105) (end 210.765 73.105) (width 0.2) (layer "F.Cu") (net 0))
 (segment (start 211.465 73.573629) (end 211.465 105.13) (width 0.2) (layer "F.Cu") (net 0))
 (segment (start 218.09 115.23) (end 212.965 110.105) (width 0.2) (layer "F.Cu") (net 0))
 (segment (start 221.65 116.52) (end 219.265 118.905) (width 0.2) (layer "F.Cu") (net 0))
 (segment (start 194.95 122.43) (end 197.115 122.43) (width 0.2) (layer "F.Cu") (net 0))
 (segment (start 210.425 110.105) (end 210.425 113.645) (width 0.2) (layer "F.Cu") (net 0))
 (segment (start 219.265 118.905) (end 219.24 118.93) (width 0.2) (layer "F.Cu") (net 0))
 (segment (start 210.996371 73.105) (end 211.465 73.573629) (width 0.2) (layer "F.Cu") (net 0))
 (segment (start 211.465 105.13) (end 210.615 105.98) (width 0.2) (layer "F.Cu") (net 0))
 (segment (start 203.465 118.48) (end 203.465 118.505) (width 0.2) (layer "F.Cu") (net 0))
 (segment (start 199.13 111.015) (end 204.315 105.83) (width 0.2) (layer "F.Cu") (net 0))
 (segment (start 193.95 121.43) (end 194.95 122.43) (width 0.2) (layer "F.Cu") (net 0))
 (segment (start 195.05 117.45) (end 199.03 121.43) (width 0.2) (layer "F.Cu") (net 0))
 (segment (start 205.715 116.255) (end 203.49 118.48) (width 0.2) (layer "F.Cu") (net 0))
 (segment (start 204.315 105.83) (end 208.69 105.83) (width 0.2) (layer "F.Cu") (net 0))
 (via (at 210.59 105.98) (size 0.6) (drill 0.3) (layers "F.Cu" "B.Cu") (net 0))
 (via (at 216.065 120.605) (size 0.6) (drill 0.3) (layers "F.Cu" "B.Cu") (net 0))
 (via (at 219.265 118.905) (size 0.6) (drill 0.3) (layers "F.Cu" "B.Cu") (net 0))
 (via (at 200.49 124.055) (size 0.6) (drill 0.3) (layers "F.Cu" "B.Cu") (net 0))
 (via (at 203.465 118.48) (size 0.6) (drill 0.3) (layers "F.Cu" "B.Cu") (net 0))
 (via (at 197.94 123.23) (size 0.6) (drill 0.3) (layers "F.Cu" "B.Cu") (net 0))
 (segment (start 213.205 73.905) (end 213.205 108.615) (width 0.2) (layer "B.Cu") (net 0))
 (segment (start 202.065 112.253629) (end 202.065 122.305) (width 0.2) (layer "B.Cu") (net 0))
 (segment (start 211.035686 123.655686) (end 207.792157 123.655686) (width 0.2) (layer "B.Cu") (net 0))
 (segment (start 210.59 105.98) (end 210.425 106.145) (width 0.2) (layer "B.Cu") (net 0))
 (segment (start 202.465 118.894215) (end 202.465 112.985) (width 0.2) (layer "B.Cu") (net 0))
 (segment (start 201.405 74.38) (end 201.405 124.535) (width 0.2) (layer "B.Cu") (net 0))
 (segment (start 197.94 123.23) (end 199.69 123.23) (width 0.2) (layer "B.Cu") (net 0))
 (segment (start 195.09 120.29) (end 193.95 121.43) (width 0.2) (layer "B.Cu") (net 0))
 (segment (start 191.74 74.305) (end 191.74 113.345) (width 0.2) (layer "B.Cu") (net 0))
 (segment (start 200.49 124.055) (end 200.515 124.055) (width 0.2) (layer "B.Cu") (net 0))
 (segment (start 202.49 73.105) (end 202.288553 73.306447) (width 0.2) (layer "B.Cu") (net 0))
 (segment (start 216.065 120.605) (end 215.99 120.705) (width 0.2) (layer "B.Cu") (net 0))
 (segment (start 200.515 124.055) (end 200.515 124.055) (width 0.2) (layer "B.Cu") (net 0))
 (segment (start 210.47 125.63) (end 208.895686 124.055686) (width 0.2) (layer "B.Cu") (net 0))
 (segment (start 202.288553 73.306447) (end 201.637106 72.655) (width 0.2) (layer "B.Cu") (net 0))
 (segment (start 202.865 114.455) (end 207.215 110.105) (width 0.2) (layer "B.Cu") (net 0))
 (segment (start 202.655 73.672894) (end 202.288553 73.306447) (width 0.2) (layer "B.Cu") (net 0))
 (segment (start 202.065 122.305) (end 205.39 125.63) (width 0.2) (layer "B.Cu") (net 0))
 (segment (start 213.205 108.615) (end 208.685 113.135) (width 0.2) (layer "B.Cu") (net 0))
 (segment (start 199.69 123.23) (end 200.49 124.03) (width 0.2) (layer "B.Cu") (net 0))
 (segment (start 210.925 121.005) (end 215.55 125.63) (width 0.2) (layer "B.Cu") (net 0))
 (segment (start 201.637106 72.655) (end 195.09 79.202106) (width 0.2) (layer "B.Cu") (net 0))
 (segment (start 200.49 124.03) (end 200.49 124.055) (width 0.2) (layer "B.Cu") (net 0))
 (segment (start 207.626471 124.055686) (end 202.465 118.894215) (width 0.2) (layer "B.Cu") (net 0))
 (segment (start 208.685 113.135) (end 208.685 109.773629) (width 0.2) (layer "B.Cu") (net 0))
 (segment (start 202.865 118.728529) (end 202.865 114.455) (width 0.2) (layer "B.Cu") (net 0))
 (segment (start 202.655 74.38) (end 202.655 73.672894) (width 0.2) (layer "B.Cu") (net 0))
 (segment (start 208.216371 109.305) (end 205.013629 109.305) (width 0.2) (layer "B.Cu") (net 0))
 (segment (start 207.215 110.105) (end 207.885 110.105) (width 0.2) (layer "B.Cu") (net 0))
 (segment (start 219.265 118.905) (end 217.465 120.705) (width 0.2) (layer "B.Cu") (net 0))
 (segment (start 201.405 124.535) (end 200.31 125.63) (width 0.2) (layer "B.Cu") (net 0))
 (segment (start 210.425 106.145) (end 210.425 110.105) (width 0.2) (layer "B.Cu") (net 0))
 (segment (start 208.895686 124.055686) (end 207.626471 124.055686) (width 0.2) (layer "B.Cu") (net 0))
 (segment (start 217.465 120.705) (end 216.065 120.605) (width 0.2) (layer "B.Cu") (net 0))
 (segment (start 226.73 73.905) (end 225.93 73.105) (width 0.2) (layer "B.Cu") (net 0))
 (segment (start 225.93 73.105) (end 202.49 73.105) (width 0.2) (layer "B.Cu") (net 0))
 (segment (start 208.685 109.773629) (end 208.216371 109.305) (width 0.2) (layer "B.Cu") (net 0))
 (segment (start 203.465 118.48) (end 205.99 121.005) (width 0.2) (layer "B.Cu") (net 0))
 (segment (start 205.99 121.005) (end 210.925 121.005) (width 0.2) (layer "B.Cu") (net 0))
 (segment (start 191.74 113.345) (end 194.05 115.655) (width 0.2) (layer "B.Cu") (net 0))
 (segment (start 202.465 112.985) (end 205.345 110.105) (width 0.2) (layer "B.Cu") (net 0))
 (segment (start 205.013629 109.305) (end 202.065 112.253629) (width 0.2) (layer "B.Cu") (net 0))
 (segment (start 213.01 125.63) (end 211.035686 123.655686) (width 0.2) (layer "B.Cu") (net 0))
 (segment (start 195.09 79.202106) (end 195.09 120.29) (width 0.2) (layer "B.Cu") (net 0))
 (segment (start 207.792157 123.655686) (end 202.865 118.728529) (width 0.2) (layer "B.Cu") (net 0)))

